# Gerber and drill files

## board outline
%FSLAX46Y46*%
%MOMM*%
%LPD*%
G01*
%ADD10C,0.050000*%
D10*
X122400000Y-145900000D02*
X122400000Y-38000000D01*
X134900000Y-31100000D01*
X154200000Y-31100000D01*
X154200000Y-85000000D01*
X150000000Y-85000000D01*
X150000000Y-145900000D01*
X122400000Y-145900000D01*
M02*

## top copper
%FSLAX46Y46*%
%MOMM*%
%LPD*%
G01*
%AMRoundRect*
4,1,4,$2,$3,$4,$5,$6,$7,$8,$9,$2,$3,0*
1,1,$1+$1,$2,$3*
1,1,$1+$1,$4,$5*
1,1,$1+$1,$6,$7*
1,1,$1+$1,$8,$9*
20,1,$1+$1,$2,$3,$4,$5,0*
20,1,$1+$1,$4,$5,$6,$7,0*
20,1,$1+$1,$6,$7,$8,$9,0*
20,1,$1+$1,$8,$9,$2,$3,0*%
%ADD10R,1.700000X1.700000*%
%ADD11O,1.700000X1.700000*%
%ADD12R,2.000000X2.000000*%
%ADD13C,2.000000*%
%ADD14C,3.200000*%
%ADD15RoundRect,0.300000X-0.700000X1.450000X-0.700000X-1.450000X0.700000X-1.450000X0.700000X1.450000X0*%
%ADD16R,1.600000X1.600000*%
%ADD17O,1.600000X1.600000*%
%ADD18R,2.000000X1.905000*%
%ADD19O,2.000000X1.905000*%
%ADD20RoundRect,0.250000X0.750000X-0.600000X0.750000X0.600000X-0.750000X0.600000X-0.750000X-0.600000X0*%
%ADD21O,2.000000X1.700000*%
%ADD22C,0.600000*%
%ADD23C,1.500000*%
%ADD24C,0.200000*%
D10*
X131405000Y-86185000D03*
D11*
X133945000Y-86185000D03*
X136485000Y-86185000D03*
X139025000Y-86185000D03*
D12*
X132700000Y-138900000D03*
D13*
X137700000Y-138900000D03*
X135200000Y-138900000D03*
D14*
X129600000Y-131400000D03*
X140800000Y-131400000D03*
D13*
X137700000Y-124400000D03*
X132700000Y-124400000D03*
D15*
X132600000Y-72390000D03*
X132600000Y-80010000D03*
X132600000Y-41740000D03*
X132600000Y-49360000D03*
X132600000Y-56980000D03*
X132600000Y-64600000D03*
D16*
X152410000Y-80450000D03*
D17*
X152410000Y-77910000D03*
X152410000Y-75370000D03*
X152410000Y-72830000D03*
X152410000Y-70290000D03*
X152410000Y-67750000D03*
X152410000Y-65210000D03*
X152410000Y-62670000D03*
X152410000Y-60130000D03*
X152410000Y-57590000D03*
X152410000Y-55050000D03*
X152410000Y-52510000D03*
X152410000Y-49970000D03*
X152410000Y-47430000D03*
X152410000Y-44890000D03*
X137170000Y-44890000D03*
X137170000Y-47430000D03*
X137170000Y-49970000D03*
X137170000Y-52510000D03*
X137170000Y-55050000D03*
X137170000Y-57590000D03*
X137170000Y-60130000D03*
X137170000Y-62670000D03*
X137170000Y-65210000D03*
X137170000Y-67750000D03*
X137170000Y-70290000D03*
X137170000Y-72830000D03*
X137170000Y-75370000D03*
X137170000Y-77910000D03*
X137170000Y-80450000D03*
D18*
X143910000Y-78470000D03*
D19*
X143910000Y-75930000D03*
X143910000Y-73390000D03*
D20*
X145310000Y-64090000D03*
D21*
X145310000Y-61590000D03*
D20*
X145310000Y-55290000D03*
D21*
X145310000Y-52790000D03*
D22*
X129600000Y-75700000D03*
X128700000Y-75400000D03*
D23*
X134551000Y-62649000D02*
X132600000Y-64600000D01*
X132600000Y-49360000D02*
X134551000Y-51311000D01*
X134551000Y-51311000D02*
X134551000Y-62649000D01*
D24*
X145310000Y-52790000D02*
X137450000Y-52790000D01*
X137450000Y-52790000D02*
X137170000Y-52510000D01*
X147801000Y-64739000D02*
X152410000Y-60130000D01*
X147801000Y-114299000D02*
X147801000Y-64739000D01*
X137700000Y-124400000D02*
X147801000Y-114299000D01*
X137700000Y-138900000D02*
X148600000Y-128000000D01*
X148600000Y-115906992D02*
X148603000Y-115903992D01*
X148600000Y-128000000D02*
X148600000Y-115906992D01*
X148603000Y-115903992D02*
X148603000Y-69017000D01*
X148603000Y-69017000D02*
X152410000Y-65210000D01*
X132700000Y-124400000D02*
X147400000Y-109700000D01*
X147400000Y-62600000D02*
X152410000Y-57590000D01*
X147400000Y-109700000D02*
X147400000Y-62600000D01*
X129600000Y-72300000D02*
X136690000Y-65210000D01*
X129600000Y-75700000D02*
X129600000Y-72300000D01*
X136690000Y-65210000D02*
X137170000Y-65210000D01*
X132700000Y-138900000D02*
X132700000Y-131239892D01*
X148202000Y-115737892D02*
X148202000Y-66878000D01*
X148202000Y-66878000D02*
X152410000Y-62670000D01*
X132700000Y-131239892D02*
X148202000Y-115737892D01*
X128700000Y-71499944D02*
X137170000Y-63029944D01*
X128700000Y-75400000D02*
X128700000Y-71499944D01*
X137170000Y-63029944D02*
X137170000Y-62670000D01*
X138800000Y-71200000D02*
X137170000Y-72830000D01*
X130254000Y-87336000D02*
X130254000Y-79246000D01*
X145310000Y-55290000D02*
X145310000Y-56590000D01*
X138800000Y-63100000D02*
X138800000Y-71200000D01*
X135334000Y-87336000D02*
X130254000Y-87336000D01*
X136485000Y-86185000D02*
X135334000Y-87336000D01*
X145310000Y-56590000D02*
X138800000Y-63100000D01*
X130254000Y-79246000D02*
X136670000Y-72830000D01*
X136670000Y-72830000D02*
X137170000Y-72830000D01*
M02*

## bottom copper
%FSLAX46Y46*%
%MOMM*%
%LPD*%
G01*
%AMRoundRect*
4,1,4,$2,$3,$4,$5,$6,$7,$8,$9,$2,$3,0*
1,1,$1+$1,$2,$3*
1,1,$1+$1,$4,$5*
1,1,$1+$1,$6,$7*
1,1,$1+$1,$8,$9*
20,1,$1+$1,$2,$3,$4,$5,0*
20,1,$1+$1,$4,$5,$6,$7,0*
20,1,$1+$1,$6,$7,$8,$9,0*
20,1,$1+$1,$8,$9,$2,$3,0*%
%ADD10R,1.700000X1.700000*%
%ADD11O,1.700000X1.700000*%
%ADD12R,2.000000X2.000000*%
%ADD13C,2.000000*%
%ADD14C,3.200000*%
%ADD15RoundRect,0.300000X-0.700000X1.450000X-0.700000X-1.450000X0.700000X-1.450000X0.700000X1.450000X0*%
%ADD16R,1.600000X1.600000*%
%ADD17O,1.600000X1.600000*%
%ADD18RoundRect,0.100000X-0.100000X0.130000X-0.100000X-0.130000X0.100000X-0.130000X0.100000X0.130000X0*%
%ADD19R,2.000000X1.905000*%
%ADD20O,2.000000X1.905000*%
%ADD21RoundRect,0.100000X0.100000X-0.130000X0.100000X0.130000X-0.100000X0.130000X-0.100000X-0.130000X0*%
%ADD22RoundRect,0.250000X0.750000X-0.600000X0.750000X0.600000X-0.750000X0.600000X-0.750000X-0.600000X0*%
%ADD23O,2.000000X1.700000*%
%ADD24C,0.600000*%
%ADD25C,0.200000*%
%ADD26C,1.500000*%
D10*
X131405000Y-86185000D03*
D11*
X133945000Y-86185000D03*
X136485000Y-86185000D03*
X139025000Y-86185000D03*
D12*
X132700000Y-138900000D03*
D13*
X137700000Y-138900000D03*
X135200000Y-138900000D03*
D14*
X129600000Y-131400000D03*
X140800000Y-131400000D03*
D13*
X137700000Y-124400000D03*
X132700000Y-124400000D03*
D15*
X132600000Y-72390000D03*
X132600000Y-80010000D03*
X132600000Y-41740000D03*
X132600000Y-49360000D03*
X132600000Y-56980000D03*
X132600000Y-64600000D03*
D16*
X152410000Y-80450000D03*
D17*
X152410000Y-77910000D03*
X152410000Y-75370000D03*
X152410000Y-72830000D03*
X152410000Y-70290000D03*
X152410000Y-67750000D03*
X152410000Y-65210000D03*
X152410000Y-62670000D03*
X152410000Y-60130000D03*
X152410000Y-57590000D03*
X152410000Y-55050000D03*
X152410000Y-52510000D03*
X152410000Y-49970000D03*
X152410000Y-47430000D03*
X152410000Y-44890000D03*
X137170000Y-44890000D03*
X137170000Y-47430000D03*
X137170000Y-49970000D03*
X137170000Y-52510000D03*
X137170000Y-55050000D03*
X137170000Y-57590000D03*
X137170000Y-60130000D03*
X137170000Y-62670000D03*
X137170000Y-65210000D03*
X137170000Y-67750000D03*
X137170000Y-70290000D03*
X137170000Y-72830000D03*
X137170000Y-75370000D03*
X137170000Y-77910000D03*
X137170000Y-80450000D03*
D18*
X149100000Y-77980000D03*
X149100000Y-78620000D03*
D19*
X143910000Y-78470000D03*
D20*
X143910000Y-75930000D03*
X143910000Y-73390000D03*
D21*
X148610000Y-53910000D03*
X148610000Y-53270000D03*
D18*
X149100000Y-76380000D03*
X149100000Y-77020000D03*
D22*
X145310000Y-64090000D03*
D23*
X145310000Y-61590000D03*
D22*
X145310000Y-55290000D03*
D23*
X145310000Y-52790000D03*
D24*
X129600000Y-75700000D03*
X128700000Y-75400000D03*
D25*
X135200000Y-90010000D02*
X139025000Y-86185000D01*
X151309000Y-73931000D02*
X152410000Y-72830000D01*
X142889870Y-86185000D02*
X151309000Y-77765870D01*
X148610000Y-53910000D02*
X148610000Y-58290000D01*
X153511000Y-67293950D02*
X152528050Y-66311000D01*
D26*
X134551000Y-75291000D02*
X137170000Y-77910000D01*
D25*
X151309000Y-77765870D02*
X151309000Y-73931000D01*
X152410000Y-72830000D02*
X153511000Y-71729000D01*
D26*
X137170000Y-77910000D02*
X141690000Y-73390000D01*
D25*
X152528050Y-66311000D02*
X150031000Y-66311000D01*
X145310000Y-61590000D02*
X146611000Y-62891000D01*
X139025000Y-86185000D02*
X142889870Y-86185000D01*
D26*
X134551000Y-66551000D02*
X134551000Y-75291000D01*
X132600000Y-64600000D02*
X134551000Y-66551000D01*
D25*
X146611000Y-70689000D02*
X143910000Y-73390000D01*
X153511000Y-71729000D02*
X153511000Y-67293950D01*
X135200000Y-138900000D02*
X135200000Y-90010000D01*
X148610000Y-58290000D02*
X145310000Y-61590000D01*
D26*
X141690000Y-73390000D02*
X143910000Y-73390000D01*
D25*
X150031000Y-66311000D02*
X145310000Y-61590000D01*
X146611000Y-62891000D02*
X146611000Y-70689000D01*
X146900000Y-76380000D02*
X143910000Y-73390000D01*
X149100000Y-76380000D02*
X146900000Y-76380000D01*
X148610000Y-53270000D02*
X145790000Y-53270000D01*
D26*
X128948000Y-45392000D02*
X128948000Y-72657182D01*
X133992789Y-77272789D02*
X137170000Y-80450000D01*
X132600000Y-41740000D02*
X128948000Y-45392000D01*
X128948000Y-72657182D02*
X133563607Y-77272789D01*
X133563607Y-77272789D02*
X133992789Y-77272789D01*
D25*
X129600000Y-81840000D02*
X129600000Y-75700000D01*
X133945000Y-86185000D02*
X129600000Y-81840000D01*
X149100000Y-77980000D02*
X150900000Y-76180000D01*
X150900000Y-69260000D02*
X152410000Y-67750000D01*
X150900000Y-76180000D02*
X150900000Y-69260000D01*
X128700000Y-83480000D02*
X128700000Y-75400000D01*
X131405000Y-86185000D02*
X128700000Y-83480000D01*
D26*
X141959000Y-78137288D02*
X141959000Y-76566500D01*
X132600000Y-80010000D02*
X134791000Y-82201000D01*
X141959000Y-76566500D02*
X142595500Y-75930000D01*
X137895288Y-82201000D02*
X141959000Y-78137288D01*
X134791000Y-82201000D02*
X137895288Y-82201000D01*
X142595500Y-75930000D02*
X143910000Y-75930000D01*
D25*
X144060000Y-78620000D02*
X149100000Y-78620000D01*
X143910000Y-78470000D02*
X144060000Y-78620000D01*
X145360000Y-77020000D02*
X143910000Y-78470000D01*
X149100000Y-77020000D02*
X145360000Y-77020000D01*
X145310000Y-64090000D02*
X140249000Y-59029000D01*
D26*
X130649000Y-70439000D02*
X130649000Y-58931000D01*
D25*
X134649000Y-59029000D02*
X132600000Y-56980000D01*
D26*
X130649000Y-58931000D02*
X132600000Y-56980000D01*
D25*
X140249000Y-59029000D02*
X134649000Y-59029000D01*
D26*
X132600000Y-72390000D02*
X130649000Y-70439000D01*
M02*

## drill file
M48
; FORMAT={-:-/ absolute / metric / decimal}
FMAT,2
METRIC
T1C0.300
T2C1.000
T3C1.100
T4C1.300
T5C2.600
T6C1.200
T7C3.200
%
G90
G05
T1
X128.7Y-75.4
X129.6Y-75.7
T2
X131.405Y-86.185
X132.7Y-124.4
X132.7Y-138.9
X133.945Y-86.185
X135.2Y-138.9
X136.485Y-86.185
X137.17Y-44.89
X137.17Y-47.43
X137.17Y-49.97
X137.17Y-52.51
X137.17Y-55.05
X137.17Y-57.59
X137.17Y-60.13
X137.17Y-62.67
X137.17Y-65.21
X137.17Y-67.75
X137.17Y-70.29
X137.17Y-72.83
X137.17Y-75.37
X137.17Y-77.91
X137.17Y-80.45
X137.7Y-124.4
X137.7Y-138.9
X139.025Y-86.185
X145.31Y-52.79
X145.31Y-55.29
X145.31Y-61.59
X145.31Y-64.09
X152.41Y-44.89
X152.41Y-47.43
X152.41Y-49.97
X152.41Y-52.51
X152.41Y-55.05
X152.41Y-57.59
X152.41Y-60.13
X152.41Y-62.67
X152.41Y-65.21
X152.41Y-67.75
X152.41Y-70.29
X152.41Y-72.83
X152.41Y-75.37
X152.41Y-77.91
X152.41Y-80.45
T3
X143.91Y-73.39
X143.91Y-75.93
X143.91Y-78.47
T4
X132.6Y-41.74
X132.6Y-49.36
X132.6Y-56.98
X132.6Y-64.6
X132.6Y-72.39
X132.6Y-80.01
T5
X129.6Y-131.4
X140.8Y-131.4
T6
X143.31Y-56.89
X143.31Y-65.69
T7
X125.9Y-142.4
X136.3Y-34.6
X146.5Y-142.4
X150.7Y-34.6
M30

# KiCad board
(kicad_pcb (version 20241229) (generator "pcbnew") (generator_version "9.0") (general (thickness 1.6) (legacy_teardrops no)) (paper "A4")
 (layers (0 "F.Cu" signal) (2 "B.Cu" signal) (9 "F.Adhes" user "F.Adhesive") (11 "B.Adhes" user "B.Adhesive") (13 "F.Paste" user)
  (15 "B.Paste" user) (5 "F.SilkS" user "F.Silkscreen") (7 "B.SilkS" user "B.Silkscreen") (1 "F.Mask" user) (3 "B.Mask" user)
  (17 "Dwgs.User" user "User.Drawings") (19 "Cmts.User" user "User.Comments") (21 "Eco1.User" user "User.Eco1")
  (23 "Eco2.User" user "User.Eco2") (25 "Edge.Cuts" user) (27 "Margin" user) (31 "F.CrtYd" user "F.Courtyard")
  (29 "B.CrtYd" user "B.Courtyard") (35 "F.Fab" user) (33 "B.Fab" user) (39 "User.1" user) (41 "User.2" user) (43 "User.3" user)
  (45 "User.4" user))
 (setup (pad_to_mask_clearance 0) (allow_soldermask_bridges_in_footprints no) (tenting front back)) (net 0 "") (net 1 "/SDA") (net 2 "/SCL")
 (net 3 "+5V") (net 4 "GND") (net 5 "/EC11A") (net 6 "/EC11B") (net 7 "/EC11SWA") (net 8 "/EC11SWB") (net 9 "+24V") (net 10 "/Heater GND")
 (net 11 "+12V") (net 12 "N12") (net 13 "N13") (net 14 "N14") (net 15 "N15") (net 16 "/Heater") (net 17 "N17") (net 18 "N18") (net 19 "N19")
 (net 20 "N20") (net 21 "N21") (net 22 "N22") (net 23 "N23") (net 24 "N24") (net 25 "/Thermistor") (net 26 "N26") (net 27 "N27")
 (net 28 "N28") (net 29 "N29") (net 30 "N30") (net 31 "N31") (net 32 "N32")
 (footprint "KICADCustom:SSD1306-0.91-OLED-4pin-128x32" (layer "F.Cu") (at 129.215 122.685 90)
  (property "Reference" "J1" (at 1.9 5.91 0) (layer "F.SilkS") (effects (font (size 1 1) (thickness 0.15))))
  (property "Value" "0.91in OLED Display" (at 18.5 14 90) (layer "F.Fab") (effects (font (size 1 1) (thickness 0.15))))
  (pad "1" thru_hole rect (at 36.5 2.19 90) (size 1.7 1.7) (drill 1) (layers "*.Cu" "*.Mask") (remove_unused_layers no) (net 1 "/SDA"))
  (pad "2" thru_hole oval (at 36.5 4.73 90) (size 1.7 1.7) (drill 1) (layers "*.Cu" "*.Mask") (remove_unused_layers no) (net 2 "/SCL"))
  (pad "3" thru_hole oval (at 36.5 7.27 90) (size 1.7 1.7) (drill 1) (layers "*.Cu" "*.Mask") (remove_unused_layers no) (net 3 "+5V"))
  (pad "4" thru_hole oval (at 36.5 9.81 90) (size 1.7 1.7) (drill 1) (layers "*.Cu" "*.Mask") (remove_unused_layers no) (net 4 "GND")))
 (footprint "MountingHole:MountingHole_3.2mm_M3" (layer "F.Cu") (at 146.5 142.4)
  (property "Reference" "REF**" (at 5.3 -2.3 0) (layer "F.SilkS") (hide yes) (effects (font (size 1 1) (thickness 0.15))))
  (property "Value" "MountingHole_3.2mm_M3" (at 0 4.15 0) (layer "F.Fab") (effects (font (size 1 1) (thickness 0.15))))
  (pad "" np_thru_hole circle (at 0 0) (size 3.2 3.2) (drill 3.2) (layers "*.Cu" "*.Mask")))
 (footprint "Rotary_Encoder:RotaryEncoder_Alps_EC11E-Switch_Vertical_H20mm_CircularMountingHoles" (layer "F.Cu") (at 132.7 138.9 90)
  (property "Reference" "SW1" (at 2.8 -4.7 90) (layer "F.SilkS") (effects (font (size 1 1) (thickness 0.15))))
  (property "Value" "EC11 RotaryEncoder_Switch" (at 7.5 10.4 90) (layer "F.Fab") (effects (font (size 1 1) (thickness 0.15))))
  (pad "A" thru_hole rect (at 0 0 90) (size 2 2) (drill 1) (layers "*.Cu" "*.Mask") (remove_unused_layers no) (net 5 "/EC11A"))
  (pad "B" thru_hole circle (at 0 5 90) (size 2 2) (drill 1) (layers "*.Cu" "*.Mask") (remove_unused_layers no) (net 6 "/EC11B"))
  (pad "C" thru_hole circle (at 0 2.5 90) (size 2 2) (drill 1) (layers "*.Cu" "*.Mask") (remove_unused_layers no) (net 4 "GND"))
  (pad "MP" thru_hole circle (at 7.5 -3.1 90) (size 3.2 3.2) (drill 2.6) (layers "*.Cu" "*.Mask") (remove_unused_layers no))
  (pad "MP" thru_hole circle (at 7.5 8.1 90) (size 3.2 3.2) (drill 2.6) (layers "*.Cu" "*.Mask") (remove_unused_layers no))
  (pad "S1" thru_hole circle (at 14.5 5 90) (size 2 2) (drill 1) (layers "*.Cu" "*.Mask") (remove_unused_layers no) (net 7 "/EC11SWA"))
  (pad "S2" thru_hole circle (at 14.5 0 90) (size 2 2) (drill 1) (layers "*.Cu" "*.Mask") (remove_unused_layers no) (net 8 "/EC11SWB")))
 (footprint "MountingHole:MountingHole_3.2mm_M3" (layer "F.Cu") (at 136.3 34.6)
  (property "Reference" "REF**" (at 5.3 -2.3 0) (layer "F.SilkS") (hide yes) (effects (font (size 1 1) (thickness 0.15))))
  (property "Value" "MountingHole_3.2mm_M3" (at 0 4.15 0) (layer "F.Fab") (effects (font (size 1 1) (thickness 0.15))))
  (pad "" np_thru_hole circle (at 0 0) (size 3.2 3.2) (drill 3.2) (layers "*.Cu" "*.Mask")))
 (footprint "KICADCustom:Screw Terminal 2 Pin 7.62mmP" (layer "F.Cu") (at 132.6 72.39 -90)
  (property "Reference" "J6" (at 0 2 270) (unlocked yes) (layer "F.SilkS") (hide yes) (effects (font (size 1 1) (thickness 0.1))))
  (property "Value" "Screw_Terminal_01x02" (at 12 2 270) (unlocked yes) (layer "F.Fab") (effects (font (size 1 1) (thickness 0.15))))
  (pad "1" thru_hole roundrect (at 0 0 270) (size 3.5 2) (drill 1.3) (layers "*.Cu" "*.Mask") (remove_unused_layers no)
   (roundrect_rratio 0.15) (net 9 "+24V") (thermal_bridge_angle 45))
  (pad "2" thru_hole roundrect (at 7.62 0 270) (size 3.5 2) (drill 1.3) (layers "*.Cu" "*.Mask") (remove_unused_layers no)
   (roundrect_rratio 0.15) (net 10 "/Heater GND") (thermal_bridge_angle 45)))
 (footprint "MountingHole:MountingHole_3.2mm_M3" (layer "F.Cu") (at 150.7 34.6)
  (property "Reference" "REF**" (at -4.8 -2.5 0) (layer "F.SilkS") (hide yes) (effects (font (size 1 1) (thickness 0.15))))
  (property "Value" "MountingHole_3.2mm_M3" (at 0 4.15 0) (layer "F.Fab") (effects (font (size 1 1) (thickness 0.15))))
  (pad "" np_thru_hole circle (at 0 0) (size 3.2 3.2) (drill 3.2) (layers "*.Cu" "*.Mask")))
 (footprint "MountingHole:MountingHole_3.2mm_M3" (layer "F.Cu") (at 125.9 142.4)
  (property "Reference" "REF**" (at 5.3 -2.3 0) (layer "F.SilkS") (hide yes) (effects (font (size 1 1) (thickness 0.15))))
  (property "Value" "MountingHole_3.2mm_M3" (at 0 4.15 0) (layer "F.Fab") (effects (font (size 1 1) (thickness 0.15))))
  (pad "" np_thru_hole circle (at 0 0) (size 3.2 3.2) (drill 3.2) (layers "*.Cu" "*.Mask")))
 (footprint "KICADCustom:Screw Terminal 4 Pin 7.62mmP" (layer "F.Cu") (at 132.6 41.74 -90)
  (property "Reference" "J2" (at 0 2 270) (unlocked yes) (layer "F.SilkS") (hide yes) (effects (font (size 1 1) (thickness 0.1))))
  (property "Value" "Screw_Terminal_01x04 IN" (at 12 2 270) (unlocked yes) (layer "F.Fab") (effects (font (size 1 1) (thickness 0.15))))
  (pad "1" thru_hole roundrect (at 0 0 270) (size 3.5 2) (drill 1.3) (layers "*.Cu" "*.Mask") (remove_unused_layers no)
   (roundrect_rratio 0.15) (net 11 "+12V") (thermal_bridge_angle 45))
  (pad "2" thru_hole roundrect (at 7.62 0 270) (size 3.5 2) (drill 1.3) (layers "*.Cu" "*.Mask") (remove_unused_layers no)
   (roundrect_rratio 0.15) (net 4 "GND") (thermal_bridge_angle 45))
  (pad "3" thru_hole roundrect (at 15.24 0 270) (size 3.5 2) (drill 1.3) (layers "*.Cu" "*.Mask") (remove_unused_layers no)
   (roundrect_rratio 0.15) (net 9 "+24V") (thermal_bridge_angle 45))
  (pad "4" thru_hole roundrect (at 22.86 0 270) (size 3.5 2) (drill 1.3) (layers "*.Cu" "*.Mask") (remove_unused_layers no)
   (roundrect_rratio 0.15) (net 4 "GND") (thermal_bridge_angle 45)))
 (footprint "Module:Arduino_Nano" (layer "F.Cu") (at 152.41 80.45 180)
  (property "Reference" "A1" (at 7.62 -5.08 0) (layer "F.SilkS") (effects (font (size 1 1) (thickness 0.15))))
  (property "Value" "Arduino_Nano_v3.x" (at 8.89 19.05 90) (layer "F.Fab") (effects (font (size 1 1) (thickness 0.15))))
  (pad "1" thru_hole rect (at 0 0 180) (size 1.6 1.6) (drill 1) (layers "*.Cu" "*.Mask") (remove_unused_layers no) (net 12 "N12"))
  (pad "2" thru_hole oval (at 0 2.54 180) (size 1.6 1.6) (drill 1) (layers "*.Cu" "*.Mask") (remove_unused_layers no) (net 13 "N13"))
  (pad "3" thru_hole oval (at 0 5.08 180) (size 1.6 1.6) (drill 1) (layers "*.Cu" "*.Mask") (remove_unused_layers no) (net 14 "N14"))
  (pad "4" thru_hole oval (at 0 7.62 180) (size 1.6 1.6) (drill 1) (layers "*.Cu" "*.Mask") (remove_unused_layers no) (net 4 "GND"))
  (pad "5" thru_hole oval (at 0 10.16 180) (size 1.6 1.6) (drill 1) (layers "*.Cu" "*.Mask") (remove_unused_layers no) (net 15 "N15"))
  (pad "6" thru_hole oval (at 0 12.7 180) (size 1.6 1.6) (drill 1) (layers "*.Cu" "*.Mask") (remove_unused_layers no) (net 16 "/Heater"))
  (pad "7" thru_hole oval (at 0 15.24 180) (size 1.6 1.6) (drill 1) (layers "*.Cu" "*.Mask") (remove_unused_layers no) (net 6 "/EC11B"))
  (pad "8" thru_hole oval (at 0 17.78 180) (size 1.6 1.6) (drill 1) (layers "*.Cu" "*.Mask") (remove_unused_layers no) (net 5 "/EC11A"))
  (pad "9" thru_hole oval (at 0 20.32 180) (size 1.6 1.6) (drill 1) (layers "*.Cu" "*.Mask") (remove_unused_layers no) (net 7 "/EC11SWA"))
  (pad "10" thru_hole oval (at 0 22.86 180) (size 1.6 1.6) (drill 1) (layers "*.Cu" "*.Mask") (remove_unused_layers no) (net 8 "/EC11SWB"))
  (pad "11" thru_hole oval (at 0 25.4 180) (size 1.6 1.6) (drill 1) (layers "*.Cu" "*.Mask") (remove_unused_layers no) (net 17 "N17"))
  (pad "12" thru_hole oval (at 0 27.94 180) (size 1.6 1.6) (drill 1) (layers "*.Cu" "*.Mask") (remove_unused_layers no) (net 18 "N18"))
  (pad "13" thru_hole oval (at 0 30.48 180) (size 1.6 1.6) (drill 1) (layers "*.Cu" "*.Mask") (remove_unused_layers no) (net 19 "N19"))
  (pad "14" thru_hole oval (at 0 33.02 180) (size 1.6 1.6) (drill 1) (layers "*.Cu" "*.Mask") (remove_unused_layers no) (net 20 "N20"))
  (pad "15" thru_hole oval (at 0 35.56 180) (size 1.6 1.6) (drill 1) (layers "*.Cu" "*.Mask") (remove_unused_layers no) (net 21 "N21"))
  (pad "16" thru_hole oval (at 15.24 35.56 180) (size 1.6 1.6) (drill 1) (layers "*.Cu" "*.Mask") (remove_unused_layers no) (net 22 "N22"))
  (pad "17" thru_hole oval (at 15.24 33.02 180) (size 1.6 1.6) (drill 1) (layers "*.Cu" "*.Mask") (remove_unused_layers no) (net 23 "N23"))
  (pad "18" thru_hole oval (at 15.24 30.48 180) (size 1.6 1.6) (drill 1) (layers "*.Cu" "*.Mask") (remove_unused_layers no) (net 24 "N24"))
  (pad "19" thru_hole oval (at 15.24 27.94 180) (size 1.6 1.6) (drill 1) (layers "*.Cu" "*.Mask") (remove_unused_layers no)
   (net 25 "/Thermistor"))
  (pad "20" thru_hole oval (at 15.24 25.4 180) (size 1.6 1.6) (drill 1) (layers "*.Cu" "*.Mask") (remove_unused_layers no) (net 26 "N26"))
  (pad "21" thru_hole oval (at 15.24 22.86 180) (size 1.6 1.6) (drill 1) (layers "*.Cu" "*.Mask") (remove_unused_layers no) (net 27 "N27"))
  (pad "22" thru_hole oval (at 15.24 20.32 180) (size 1.6 1.6) (drill 1) (layers "*.Cu" "*.Mask") (remove_unused_layers no) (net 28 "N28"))
  (pad "23" thru_hole oval (at 15.24 17.78 180) (size 1.6 1.6) (drill 1) (layers "*.Cu" "*.Mask") (remove_unused_layers no) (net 1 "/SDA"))
  (pad "24" thru_hole oval (at 15.24 15.24 180) (size 1.6 1.6) (drill 1) (layers "*.Cu" "*.Mask") (remove_unused_layers no) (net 2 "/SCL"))
  (pad "25" thru_hole oval (at 15.24 12.7 180) (size 1.6 1.6) (drill 1) (layers "*.Cu" "*.Mask") (remove_unused_layers no) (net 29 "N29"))
  (pad "26" thru_hole oval (at 15.24 10.16 180) (size 1.6 1.6) (drill 1) (layers "*.Cu" "*.Mask") (remove_unused_layers no) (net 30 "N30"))
  (pad "27" thru_hole oval (at 15.24 7.62 180) (size 1.6 1.6) (drill 1) (layers "*.Cu" "*.Mask") (remove_unused_layers no) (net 3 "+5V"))
  (pad "28" thru_hole oval (at 15.24 5.08 180) (size 1.6 1.6) (drill 1) (layers "*.Cu" "*.Mask") (remove_unused_layers no) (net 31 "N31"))
  (pad "29" thru_hole oval (at 15.24 2.54 180) (size 1.6 1.6) (drill 1) (layers "*.Cu" "*.Mask") (remove_unused_layers no) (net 4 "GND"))
  (pad "30" thru_hole oval (at 15.24 0 180) (size 1.6 1.6) (drill 1) (layers "*.Cu" "*.Mask") (remove_unused_layers no) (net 11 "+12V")))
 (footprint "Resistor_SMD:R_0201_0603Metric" (layer "B.Cu") (at 149.1 78.3 -90)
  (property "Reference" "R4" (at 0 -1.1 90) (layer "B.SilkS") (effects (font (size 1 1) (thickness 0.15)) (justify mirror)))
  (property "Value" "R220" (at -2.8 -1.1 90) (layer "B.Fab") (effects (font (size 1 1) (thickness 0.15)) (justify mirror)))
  (pad "" smd roundrect (at -0.345 0 270) (size 0.318 0.36) (layers "B.Paste") (roundrect_rratio 0.25))
  (pad "" smd roundrect (at 0.345 0 270) (size 0.318 0.36) (layers "B.Paste") (roundrect_rratio 0.25))
  (pad "1" smd roundrect (at -0.32 0 270) (size 0.46 0.4) (layers "B.Cu" "B.Mask") (roundrect_rratio 0.25) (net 16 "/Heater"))
  (pad "2" smd roundrect (at 0.32 0 270) (size 0.46 0.4) (layers "B.Cu" "B.Mask") (roundrect_rratio 0.25) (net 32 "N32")))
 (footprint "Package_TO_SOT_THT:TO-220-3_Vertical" (layer "B.Cu") (at 143.91 78.47 90)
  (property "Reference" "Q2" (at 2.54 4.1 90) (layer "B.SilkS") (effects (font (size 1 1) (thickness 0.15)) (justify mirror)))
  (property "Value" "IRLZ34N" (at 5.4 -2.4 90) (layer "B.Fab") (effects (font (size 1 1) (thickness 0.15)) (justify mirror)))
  (pad "1" thru_hole rect (at 0 0 90) (size 1.905 2) (drill 1.1) (layers "*.Cu" "*.Mask") (remove_unused_layers no) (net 32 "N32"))
  (pad "2" thru_hole oval (at 2.54 0 90) (size 1.905 2) (drill 1.1) (layers "*.Cu" "*.Mask") (remove_unused_layers no)
   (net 10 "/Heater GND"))
  (pad "3" thru_hole oval (at 5.08 0 90) (size 1.905 2) (drill 1.1) (layers "*.Cu" "*.Mask") (remove_unused_layers no) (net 4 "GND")))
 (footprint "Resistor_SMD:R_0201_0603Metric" (layer "B.Cu") (at 148.61 53.59 90)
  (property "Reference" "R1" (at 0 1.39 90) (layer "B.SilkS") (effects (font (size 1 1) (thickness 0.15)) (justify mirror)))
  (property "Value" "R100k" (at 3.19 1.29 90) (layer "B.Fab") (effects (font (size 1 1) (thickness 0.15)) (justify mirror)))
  (pad "" smd roundrect (at -0.345 0 90) (size 0.318 0.36) (layers "B.Paste") (roundrect_rratio 0.25))
  (pad "" smd roundrect (at 0.345 0 90) (size 0.318 0.36) (layers "B.Paste") (roundrect_rratio 0.25))
  (pad "1" smd roundrect (at -0.32 0 90) (size 0.46 0.4) (layers "B.Cu" "B.Mask") (roundrect_rratio 0.25) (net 4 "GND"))
  (pad "2" smd roundrect (at 0.32 0 90) (size 0.46 0.4) (layers "B.Cu" "B.Mask") (roundrect_rratio 0.25) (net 25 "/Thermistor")))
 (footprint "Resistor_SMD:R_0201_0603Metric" (layer "B.Cu") (at 149.1 76.7 -90)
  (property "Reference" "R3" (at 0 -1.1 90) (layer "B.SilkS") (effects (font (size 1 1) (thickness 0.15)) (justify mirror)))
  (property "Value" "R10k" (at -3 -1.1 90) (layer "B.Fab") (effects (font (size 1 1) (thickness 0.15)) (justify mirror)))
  (pad "" smd roundrect (at -0.345 0 270) (size 0.318 0.36) (layers "B.Paste") (roundrect_rratio 0.25))
  (pad "" smd roundrect (at 0.345 0 270) (size 0.318 0.36) (layers "B.Paste") (roundrect_rratio 0.25))
  (pad "1" smd roundrect (at -0.32 0 270) (size 0.46 0.4) (layers "B.Cu" "B.Mask") (roundrect_rratio 0.25) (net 4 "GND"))
  (pad "2" smd roundrect (at 0.32 0 270) (size 0.46 0.4) (layers "B.Cu" "B.Mask") (roundrect_rratio 0.25) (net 32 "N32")))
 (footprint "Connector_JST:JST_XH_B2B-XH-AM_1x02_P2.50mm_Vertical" (layer "B.Cu") (at 145.31 64.09 90)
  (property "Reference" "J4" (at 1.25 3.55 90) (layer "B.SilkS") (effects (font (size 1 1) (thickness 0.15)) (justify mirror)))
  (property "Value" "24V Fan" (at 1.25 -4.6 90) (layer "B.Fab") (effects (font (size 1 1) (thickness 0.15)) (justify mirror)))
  (pad "" np_thru_hole circle (at -1.6 -2 90) (size 1.2 1.2) (drill 1.2) (layers "*.Cu" "*.Mask"))
  (pad "1" thru_hole roundrect (at 0 0 90) (size 1.7 2) (drill 1) (layers "*.Cu" "*.Mask") (remove_unused_layers no)
   (roundrect_rratio 0.147059) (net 9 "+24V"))
  (pad "2" thru_hole oval (at 2.5 0 90) (size 1.7 2) (drill 1) (layers "*.Cu" "*.Mask") (remove_unused_layers no) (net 4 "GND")))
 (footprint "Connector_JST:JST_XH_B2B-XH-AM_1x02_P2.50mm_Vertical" (layer "B.Cu") (at 145.31 55.29 90)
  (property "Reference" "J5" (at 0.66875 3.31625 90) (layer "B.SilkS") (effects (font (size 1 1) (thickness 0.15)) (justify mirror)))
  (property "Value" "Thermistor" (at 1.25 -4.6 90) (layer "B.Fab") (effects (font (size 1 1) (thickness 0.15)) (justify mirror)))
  (pad "" np_thru_hole circle (at -1.6 -2 90) (size 1.2 1.2) (drill 1.2) (layers "*.Cu" "*.Mask"))
  (pad "1" thru_hole roundrect (at 0 0 90) (size 1.7 2) (drill 1) (layers "*.Cu" "*.Mask") (remove_unused_layers no)
   (roundrect_rratio 0.147059) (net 3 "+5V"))
  (pad "2" thru_hole oval (at 2.5 0 90) (size 1.7 2) (drill 1) (layers "*.Cu" "*.Mask") (remove_unused_layers no) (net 25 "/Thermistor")))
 (gr_poly
  (pts (xy 122.4 145.9) (xy 122.4 38) (xy 134.9 31.1) (xy 154.2 31.1) (xy 154.2 85) (xy 150 85) (xy 150 145.9))
  (stroke (width 0.05) (type solid)) (fill no) (layer "Edge.Cuts"))
 (segment (start 134.551 62.649) (end 132.6 64.6) (width 1.5) (layer "F.Cu") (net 4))
 (segment (start 132.6 49.36) (end 134.551 51.311) (width 1.5) (layer "F.Cu") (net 4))
 (segment (start 134.551 51.311) (end 134.551 62.649) (width 1.5) (layer "F.Cu") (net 4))
 (segment (start 135.2 90.01) (end 139.025 86.185) (width 0.2) (layer "B.Cu") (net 4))
 (segment (start 151.309 73.931) (end 152.41 72.83) (width 0.2) (layer "B.Cu") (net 4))
 (segment (start 142.88987 86.185) (end 151.309 77.76587) (width 0.2) (layer "B.Cu") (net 4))
 (segment (start 148.61 53.91) (end 148.61 58.29) (width 0.2) (layer "B.Cu") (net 4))
 (segment (start 153.511 67.29395) (end 152.52805 66.311) (width 0.2) (layer "B.Cu") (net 4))
 (segment (start 134.551 75.291) (end 137.17 77.91) (width 1.5) (layer "B.Cu") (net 4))
 (segment (start 151.309 77.76587) (end 151.309 73.931) (width 0.2) (layer "B.Cu") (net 4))
 (segment (start 152.41 72.83) (end 153.511 71.729) (width 0.2) (layer "B.Cu") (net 4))
 (segment (start 137.17 77.91) (end 141.69 73.39) (width 1.5) (layer "B.Cu") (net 4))
 (segment (start 152.52805 66.311) (end 150.031 66.311) (width 0.2) (layer "B.Cu") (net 4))
 (segment (start 145.31 61.59) (end 146.611 62.891) (width 0.2) (layer "B.Cu") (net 4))
 (segment (start 139.025 86.185) (end 142.88987 86.185) (width 0.2) (layer "B.Cu") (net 4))
 (segment (start 134.551 66.551) (end 134.551 75.291) (width 1.5) (layer "B.Cu") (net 4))
 (segment (start 132.6 64.6) (end 134.551 66.551) (width 1.5) (layer "B.Cu") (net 4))
 (segment (start 146.611 70.689) (end 143.91 73.39) (width 0.2) (layer "B.Cu") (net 4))
 (segment (start 153.511 71.729) (end 153.511 67.29395) (width 0.2) (layer "B.Cu") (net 4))
 (segment (start 135.2 138.9) (end 135.2 90.01) (width 0.2) (layer "B.Cu") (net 4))
 (segment (start 148.61 58.29) (end 145.31 61.59) (width 0.2) (layer "B.Cu") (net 4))
 (segment (start 141.69 73.39) (end 143.91 73.39) (width 1.5) (layer "B.Cu") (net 4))
 (segment (start 150.031 66.311) (end 145.31 61.59) (width 0.2) (layer "B.Cu") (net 4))
 (segment (start 146.611 62.891) (end 146.611 70.689) (width 0.2) (layer "B.Cu") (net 4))
 (segment (start 146.9 76.38) (end 143.91 73.39) (width 0.2) (layer "B.Cu") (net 4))
 (segment (start 149.1 76.38) (end 146.9 76.38) (width 0.2) (layer "B.Cu") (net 4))
 (segment (start 145.31 52.79) (end 137.45 52.79) (width 0.2) (layer "F.Cu") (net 25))
 (segment (start 137.45 52.79) (end 137.17 52.51) (width 0.2) (layer "F.Cu") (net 25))
 (segment (start 148.61 53.27) (end 145.79 53.27) (width 0.2) (layer "B.Cu") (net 25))
 (segment (start 147.801 64.739) (end 152.41 60.13) (width 0.2) (layer "F.Cu") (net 7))
 (segment (start 147.801 114.299) (end 147.801 64.739) (width 0.2) (layer "F.Cu") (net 7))
 (segment (start 137.7 124.4) (end 147.801 114.299) (width 0.2) (layer "F.Cu") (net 7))
 (segment (start 137.7 138.9) (end 148.6 128) (width 0.2) (layer "F.Cu") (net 6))
 (segment (start 148.6 115.906992) (end 148.603 115.903992) (width 0.2) (layer "F.Cu") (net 6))
 (segment (start 148.6 128) (end 148.6 115.906992) (width 0.2) (layer "F.Cu") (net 6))
 (segment (start 148.603 115.903992) (end 148.603 69.017) (width 0.2) (layer "F.Cu") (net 6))
 (segment (start 148.603 69.017) (end 152.41 65.21) (width 0.2) (layer "F.Cu") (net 6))
 (segment (start 132.7 124.4) (end 147.4 109.7) (width 0.2) (layer "F.Cu") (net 8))
 (segment (start 147.4 62.6) (end 152.41 57.59) (width 0.2) (layer "F.Cu") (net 8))
 (segment (start 147.4 109.7) (end 147.4 62.6) (width 0.2) (layer "F.Cu") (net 8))
 (segment (start 128.948 45.392) (end 128.948 72.657182) (width 1.5) (layer "B.Cu") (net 11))
 (segment (start 133.992789 77.272789) (end 137.17 80.45) (width 1.5) (layer "B.Cu") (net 11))
 (segment (start 132.6 41.74) (end 128.948 45.392) (width 1.5) (layer "B.Cu") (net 11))
 (segment (start 128.948 72.657182) (end 133.563607 77.272789) (width 1.5) (layer "B.Cu") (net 11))
 (segment (start 133.563607 77.272789) (end 133.992789 77.272789) (width 1.5) (layer "B.Cu") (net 11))
 (segment (start 129.6 72.3) (end 136.69 65.21) (width 0.2) (layer "F.Cu") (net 2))
 (segment (start 129.6 75.7) (end 129.6 72.3) (width 0.2) (layer "F.Cu") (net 2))
 (segment (start 136.69 65.21) (end 137.17 65.21) (width 0.2) (layer "F.Cu") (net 2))
 (via (at 129.6 75.7) (size 0.6) (drill 0.3) (layers "F.Cu" "B.Cu") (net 2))
 (segment (start 129.6 81.84) (end 129.6 75.7) (width 0.2) (layer "B.Cu") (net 2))
 (segment (start 133.945 86.185) (end 129.6 81.84) (width 0.2) (layer "B.Cu") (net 2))
 (segment (start 132.7 138.9) (end 132.7 131.239892) (width 0.2) (layer "F.Cu") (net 5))
 (segment (start 148.202 115.737892) (end 148.202 66.878) (width 0.2) (layer "F.Cu") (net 5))
 (segment (start 148.202 66.878) (end 152.41 62.67) (width 0.2) (layer "F.Cu") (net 5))
 (segment (start 132.7 131.239892) (end 148.202 115.737892) (width 0.2) (layer "F.Cu") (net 5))
 (segment (start 149.1 77.98) (end 150.9 76.18) (width 0.2) (layer "B.Cu") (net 16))
 (segment (start 150.9 69.26) (end 152.41 67.75) (width 0.2) (layer "B.Cu") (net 16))
 (segment (start 150.9 76.18) (end 150.9 69.26) (width 0.2) (layer "B.Cu") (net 16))
 (segment (start 128.7 71.499944) (end 137.17 63.029944) (width 0.2) (layer "F.Cu") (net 1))
 (segment (start 128.7 75.4) (end 128.7 71.499944) (width 0.2) (layer "F.Cu") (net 1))
 (segment (start 137.17 63.029944) (end 137.17 62.67) (width 0.2) (layer "F.Cu") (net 1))
 (via (at 128.7 75.4) (size 0.6) (drill 0.3) (layers "F.Cu" "B.Cu") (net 1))
 (segment (start 128.7 83.48) (end 128.7 75.4) (width 0.2) (layer "B.Cu") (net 1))
 (segment (start 131.405 86.185) (end 128.7 83.48) (width 0.2) (layer "B.Cu") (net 1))
 (segment (start 138.8 71.2) (end 137.17 72.83) (width 0.2) (layer "F.Cu") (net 3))
 (segment (start 130.254 87.336) (end 130.254 79.246) (width 0.2) (layer "F.Cu") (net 3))
 (segment (start 145.31 55.29) (end 145.31 56.59) (width 0.2) (layer "F.Cu") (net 3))
 (segment (start 138.8 63.1) (end 138.8 71.2) (width 0.2) (layer "F.Cu") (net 3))
 (segment (start 135.334 87.336) (end 130.254 87.336) (width 0.2) (layer "F.Cu") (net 3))
 (segment (start 136.485 86.185) (end 135.334 87.336) (width 0.2) (layer "F.Cu") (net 3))
 (segment (start 145.31 56.59) (end 138.8 63.1) (width 0.2) (layer "F.Cu") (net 3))
 (segment (start 130.254 79.246) (end 136.67 72.83) (width 0.2) (layer "F.Cu") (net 3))
 (segment (start 136.67 72.83) (end 137.17 72.83) (width 0.2) (layer "F.Cu") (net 3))
 (segment (start 141.959 78.137288) (end 141.959 76.5665) (width 1.5) (layer "B.Cu") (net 10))
 (segment (start 132.6 80.01) (end 134.791 82.201) (width 1.5) (layer "B.Cu") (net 10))
 (segment (start 141.959 76.5665) (end 142.5955 75.93) (width 1.5) (layer "B.Cu") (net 10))
 (segment (start 137.895288 82.201) (end 141.959 78.137288) (width 1.5) (layer "B.Cu") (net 10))
 (segment (start 134.791 82.201) (end 137.895288 82.201) (width 1.5) (layer "B.Cu") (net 10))
 (segment (start 142.5955 75.93) (end 143.91 75.93) (width 1.5) (layer "B.Cu") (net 10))
 (segment (start 144.06 78.62) (end 149.1 78.62) (width 0.2) (layer "B.Cu") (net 32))
 (segment (start 143.91 78.47) (end 144.06 78.62) (width 0.2) (layer "B.Cu") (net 32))
 (segment (start 145.36 77.02) (end 143.91 78.47) (width 0.2) (layer "B.Cu") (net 32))
 (segment (start 149.1 77.02) (end 145.36 77.02) (width 0.2) (layer "B.Cu") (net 32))
 (segment (start 145.31 64.09) (end 140.249 59.029) (width 0.2) (layer "B.Cu") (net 9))
 (segment (start 130.649 70.439) (end 130.649 58.931) (width 1.5) (layer "B.Cu") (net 9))
 (segment (start 134.649 59.029) (end 132.6 56.98) (width 0.2) (layer "B.Cu") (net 9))
 (segment (start 130.649 58.931) (end 132.6 56.98) (width 1.5) (layer "B.Cu") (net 9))
 (segment (start 140.249 59.029) (end 134.649 59.029) (width 0.2) (layer "B.Cu") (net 9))
 (segment (start 132.6 72.39) (end 130.649 70.439) (width 1.5) (layer "B.Cu") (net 9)))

